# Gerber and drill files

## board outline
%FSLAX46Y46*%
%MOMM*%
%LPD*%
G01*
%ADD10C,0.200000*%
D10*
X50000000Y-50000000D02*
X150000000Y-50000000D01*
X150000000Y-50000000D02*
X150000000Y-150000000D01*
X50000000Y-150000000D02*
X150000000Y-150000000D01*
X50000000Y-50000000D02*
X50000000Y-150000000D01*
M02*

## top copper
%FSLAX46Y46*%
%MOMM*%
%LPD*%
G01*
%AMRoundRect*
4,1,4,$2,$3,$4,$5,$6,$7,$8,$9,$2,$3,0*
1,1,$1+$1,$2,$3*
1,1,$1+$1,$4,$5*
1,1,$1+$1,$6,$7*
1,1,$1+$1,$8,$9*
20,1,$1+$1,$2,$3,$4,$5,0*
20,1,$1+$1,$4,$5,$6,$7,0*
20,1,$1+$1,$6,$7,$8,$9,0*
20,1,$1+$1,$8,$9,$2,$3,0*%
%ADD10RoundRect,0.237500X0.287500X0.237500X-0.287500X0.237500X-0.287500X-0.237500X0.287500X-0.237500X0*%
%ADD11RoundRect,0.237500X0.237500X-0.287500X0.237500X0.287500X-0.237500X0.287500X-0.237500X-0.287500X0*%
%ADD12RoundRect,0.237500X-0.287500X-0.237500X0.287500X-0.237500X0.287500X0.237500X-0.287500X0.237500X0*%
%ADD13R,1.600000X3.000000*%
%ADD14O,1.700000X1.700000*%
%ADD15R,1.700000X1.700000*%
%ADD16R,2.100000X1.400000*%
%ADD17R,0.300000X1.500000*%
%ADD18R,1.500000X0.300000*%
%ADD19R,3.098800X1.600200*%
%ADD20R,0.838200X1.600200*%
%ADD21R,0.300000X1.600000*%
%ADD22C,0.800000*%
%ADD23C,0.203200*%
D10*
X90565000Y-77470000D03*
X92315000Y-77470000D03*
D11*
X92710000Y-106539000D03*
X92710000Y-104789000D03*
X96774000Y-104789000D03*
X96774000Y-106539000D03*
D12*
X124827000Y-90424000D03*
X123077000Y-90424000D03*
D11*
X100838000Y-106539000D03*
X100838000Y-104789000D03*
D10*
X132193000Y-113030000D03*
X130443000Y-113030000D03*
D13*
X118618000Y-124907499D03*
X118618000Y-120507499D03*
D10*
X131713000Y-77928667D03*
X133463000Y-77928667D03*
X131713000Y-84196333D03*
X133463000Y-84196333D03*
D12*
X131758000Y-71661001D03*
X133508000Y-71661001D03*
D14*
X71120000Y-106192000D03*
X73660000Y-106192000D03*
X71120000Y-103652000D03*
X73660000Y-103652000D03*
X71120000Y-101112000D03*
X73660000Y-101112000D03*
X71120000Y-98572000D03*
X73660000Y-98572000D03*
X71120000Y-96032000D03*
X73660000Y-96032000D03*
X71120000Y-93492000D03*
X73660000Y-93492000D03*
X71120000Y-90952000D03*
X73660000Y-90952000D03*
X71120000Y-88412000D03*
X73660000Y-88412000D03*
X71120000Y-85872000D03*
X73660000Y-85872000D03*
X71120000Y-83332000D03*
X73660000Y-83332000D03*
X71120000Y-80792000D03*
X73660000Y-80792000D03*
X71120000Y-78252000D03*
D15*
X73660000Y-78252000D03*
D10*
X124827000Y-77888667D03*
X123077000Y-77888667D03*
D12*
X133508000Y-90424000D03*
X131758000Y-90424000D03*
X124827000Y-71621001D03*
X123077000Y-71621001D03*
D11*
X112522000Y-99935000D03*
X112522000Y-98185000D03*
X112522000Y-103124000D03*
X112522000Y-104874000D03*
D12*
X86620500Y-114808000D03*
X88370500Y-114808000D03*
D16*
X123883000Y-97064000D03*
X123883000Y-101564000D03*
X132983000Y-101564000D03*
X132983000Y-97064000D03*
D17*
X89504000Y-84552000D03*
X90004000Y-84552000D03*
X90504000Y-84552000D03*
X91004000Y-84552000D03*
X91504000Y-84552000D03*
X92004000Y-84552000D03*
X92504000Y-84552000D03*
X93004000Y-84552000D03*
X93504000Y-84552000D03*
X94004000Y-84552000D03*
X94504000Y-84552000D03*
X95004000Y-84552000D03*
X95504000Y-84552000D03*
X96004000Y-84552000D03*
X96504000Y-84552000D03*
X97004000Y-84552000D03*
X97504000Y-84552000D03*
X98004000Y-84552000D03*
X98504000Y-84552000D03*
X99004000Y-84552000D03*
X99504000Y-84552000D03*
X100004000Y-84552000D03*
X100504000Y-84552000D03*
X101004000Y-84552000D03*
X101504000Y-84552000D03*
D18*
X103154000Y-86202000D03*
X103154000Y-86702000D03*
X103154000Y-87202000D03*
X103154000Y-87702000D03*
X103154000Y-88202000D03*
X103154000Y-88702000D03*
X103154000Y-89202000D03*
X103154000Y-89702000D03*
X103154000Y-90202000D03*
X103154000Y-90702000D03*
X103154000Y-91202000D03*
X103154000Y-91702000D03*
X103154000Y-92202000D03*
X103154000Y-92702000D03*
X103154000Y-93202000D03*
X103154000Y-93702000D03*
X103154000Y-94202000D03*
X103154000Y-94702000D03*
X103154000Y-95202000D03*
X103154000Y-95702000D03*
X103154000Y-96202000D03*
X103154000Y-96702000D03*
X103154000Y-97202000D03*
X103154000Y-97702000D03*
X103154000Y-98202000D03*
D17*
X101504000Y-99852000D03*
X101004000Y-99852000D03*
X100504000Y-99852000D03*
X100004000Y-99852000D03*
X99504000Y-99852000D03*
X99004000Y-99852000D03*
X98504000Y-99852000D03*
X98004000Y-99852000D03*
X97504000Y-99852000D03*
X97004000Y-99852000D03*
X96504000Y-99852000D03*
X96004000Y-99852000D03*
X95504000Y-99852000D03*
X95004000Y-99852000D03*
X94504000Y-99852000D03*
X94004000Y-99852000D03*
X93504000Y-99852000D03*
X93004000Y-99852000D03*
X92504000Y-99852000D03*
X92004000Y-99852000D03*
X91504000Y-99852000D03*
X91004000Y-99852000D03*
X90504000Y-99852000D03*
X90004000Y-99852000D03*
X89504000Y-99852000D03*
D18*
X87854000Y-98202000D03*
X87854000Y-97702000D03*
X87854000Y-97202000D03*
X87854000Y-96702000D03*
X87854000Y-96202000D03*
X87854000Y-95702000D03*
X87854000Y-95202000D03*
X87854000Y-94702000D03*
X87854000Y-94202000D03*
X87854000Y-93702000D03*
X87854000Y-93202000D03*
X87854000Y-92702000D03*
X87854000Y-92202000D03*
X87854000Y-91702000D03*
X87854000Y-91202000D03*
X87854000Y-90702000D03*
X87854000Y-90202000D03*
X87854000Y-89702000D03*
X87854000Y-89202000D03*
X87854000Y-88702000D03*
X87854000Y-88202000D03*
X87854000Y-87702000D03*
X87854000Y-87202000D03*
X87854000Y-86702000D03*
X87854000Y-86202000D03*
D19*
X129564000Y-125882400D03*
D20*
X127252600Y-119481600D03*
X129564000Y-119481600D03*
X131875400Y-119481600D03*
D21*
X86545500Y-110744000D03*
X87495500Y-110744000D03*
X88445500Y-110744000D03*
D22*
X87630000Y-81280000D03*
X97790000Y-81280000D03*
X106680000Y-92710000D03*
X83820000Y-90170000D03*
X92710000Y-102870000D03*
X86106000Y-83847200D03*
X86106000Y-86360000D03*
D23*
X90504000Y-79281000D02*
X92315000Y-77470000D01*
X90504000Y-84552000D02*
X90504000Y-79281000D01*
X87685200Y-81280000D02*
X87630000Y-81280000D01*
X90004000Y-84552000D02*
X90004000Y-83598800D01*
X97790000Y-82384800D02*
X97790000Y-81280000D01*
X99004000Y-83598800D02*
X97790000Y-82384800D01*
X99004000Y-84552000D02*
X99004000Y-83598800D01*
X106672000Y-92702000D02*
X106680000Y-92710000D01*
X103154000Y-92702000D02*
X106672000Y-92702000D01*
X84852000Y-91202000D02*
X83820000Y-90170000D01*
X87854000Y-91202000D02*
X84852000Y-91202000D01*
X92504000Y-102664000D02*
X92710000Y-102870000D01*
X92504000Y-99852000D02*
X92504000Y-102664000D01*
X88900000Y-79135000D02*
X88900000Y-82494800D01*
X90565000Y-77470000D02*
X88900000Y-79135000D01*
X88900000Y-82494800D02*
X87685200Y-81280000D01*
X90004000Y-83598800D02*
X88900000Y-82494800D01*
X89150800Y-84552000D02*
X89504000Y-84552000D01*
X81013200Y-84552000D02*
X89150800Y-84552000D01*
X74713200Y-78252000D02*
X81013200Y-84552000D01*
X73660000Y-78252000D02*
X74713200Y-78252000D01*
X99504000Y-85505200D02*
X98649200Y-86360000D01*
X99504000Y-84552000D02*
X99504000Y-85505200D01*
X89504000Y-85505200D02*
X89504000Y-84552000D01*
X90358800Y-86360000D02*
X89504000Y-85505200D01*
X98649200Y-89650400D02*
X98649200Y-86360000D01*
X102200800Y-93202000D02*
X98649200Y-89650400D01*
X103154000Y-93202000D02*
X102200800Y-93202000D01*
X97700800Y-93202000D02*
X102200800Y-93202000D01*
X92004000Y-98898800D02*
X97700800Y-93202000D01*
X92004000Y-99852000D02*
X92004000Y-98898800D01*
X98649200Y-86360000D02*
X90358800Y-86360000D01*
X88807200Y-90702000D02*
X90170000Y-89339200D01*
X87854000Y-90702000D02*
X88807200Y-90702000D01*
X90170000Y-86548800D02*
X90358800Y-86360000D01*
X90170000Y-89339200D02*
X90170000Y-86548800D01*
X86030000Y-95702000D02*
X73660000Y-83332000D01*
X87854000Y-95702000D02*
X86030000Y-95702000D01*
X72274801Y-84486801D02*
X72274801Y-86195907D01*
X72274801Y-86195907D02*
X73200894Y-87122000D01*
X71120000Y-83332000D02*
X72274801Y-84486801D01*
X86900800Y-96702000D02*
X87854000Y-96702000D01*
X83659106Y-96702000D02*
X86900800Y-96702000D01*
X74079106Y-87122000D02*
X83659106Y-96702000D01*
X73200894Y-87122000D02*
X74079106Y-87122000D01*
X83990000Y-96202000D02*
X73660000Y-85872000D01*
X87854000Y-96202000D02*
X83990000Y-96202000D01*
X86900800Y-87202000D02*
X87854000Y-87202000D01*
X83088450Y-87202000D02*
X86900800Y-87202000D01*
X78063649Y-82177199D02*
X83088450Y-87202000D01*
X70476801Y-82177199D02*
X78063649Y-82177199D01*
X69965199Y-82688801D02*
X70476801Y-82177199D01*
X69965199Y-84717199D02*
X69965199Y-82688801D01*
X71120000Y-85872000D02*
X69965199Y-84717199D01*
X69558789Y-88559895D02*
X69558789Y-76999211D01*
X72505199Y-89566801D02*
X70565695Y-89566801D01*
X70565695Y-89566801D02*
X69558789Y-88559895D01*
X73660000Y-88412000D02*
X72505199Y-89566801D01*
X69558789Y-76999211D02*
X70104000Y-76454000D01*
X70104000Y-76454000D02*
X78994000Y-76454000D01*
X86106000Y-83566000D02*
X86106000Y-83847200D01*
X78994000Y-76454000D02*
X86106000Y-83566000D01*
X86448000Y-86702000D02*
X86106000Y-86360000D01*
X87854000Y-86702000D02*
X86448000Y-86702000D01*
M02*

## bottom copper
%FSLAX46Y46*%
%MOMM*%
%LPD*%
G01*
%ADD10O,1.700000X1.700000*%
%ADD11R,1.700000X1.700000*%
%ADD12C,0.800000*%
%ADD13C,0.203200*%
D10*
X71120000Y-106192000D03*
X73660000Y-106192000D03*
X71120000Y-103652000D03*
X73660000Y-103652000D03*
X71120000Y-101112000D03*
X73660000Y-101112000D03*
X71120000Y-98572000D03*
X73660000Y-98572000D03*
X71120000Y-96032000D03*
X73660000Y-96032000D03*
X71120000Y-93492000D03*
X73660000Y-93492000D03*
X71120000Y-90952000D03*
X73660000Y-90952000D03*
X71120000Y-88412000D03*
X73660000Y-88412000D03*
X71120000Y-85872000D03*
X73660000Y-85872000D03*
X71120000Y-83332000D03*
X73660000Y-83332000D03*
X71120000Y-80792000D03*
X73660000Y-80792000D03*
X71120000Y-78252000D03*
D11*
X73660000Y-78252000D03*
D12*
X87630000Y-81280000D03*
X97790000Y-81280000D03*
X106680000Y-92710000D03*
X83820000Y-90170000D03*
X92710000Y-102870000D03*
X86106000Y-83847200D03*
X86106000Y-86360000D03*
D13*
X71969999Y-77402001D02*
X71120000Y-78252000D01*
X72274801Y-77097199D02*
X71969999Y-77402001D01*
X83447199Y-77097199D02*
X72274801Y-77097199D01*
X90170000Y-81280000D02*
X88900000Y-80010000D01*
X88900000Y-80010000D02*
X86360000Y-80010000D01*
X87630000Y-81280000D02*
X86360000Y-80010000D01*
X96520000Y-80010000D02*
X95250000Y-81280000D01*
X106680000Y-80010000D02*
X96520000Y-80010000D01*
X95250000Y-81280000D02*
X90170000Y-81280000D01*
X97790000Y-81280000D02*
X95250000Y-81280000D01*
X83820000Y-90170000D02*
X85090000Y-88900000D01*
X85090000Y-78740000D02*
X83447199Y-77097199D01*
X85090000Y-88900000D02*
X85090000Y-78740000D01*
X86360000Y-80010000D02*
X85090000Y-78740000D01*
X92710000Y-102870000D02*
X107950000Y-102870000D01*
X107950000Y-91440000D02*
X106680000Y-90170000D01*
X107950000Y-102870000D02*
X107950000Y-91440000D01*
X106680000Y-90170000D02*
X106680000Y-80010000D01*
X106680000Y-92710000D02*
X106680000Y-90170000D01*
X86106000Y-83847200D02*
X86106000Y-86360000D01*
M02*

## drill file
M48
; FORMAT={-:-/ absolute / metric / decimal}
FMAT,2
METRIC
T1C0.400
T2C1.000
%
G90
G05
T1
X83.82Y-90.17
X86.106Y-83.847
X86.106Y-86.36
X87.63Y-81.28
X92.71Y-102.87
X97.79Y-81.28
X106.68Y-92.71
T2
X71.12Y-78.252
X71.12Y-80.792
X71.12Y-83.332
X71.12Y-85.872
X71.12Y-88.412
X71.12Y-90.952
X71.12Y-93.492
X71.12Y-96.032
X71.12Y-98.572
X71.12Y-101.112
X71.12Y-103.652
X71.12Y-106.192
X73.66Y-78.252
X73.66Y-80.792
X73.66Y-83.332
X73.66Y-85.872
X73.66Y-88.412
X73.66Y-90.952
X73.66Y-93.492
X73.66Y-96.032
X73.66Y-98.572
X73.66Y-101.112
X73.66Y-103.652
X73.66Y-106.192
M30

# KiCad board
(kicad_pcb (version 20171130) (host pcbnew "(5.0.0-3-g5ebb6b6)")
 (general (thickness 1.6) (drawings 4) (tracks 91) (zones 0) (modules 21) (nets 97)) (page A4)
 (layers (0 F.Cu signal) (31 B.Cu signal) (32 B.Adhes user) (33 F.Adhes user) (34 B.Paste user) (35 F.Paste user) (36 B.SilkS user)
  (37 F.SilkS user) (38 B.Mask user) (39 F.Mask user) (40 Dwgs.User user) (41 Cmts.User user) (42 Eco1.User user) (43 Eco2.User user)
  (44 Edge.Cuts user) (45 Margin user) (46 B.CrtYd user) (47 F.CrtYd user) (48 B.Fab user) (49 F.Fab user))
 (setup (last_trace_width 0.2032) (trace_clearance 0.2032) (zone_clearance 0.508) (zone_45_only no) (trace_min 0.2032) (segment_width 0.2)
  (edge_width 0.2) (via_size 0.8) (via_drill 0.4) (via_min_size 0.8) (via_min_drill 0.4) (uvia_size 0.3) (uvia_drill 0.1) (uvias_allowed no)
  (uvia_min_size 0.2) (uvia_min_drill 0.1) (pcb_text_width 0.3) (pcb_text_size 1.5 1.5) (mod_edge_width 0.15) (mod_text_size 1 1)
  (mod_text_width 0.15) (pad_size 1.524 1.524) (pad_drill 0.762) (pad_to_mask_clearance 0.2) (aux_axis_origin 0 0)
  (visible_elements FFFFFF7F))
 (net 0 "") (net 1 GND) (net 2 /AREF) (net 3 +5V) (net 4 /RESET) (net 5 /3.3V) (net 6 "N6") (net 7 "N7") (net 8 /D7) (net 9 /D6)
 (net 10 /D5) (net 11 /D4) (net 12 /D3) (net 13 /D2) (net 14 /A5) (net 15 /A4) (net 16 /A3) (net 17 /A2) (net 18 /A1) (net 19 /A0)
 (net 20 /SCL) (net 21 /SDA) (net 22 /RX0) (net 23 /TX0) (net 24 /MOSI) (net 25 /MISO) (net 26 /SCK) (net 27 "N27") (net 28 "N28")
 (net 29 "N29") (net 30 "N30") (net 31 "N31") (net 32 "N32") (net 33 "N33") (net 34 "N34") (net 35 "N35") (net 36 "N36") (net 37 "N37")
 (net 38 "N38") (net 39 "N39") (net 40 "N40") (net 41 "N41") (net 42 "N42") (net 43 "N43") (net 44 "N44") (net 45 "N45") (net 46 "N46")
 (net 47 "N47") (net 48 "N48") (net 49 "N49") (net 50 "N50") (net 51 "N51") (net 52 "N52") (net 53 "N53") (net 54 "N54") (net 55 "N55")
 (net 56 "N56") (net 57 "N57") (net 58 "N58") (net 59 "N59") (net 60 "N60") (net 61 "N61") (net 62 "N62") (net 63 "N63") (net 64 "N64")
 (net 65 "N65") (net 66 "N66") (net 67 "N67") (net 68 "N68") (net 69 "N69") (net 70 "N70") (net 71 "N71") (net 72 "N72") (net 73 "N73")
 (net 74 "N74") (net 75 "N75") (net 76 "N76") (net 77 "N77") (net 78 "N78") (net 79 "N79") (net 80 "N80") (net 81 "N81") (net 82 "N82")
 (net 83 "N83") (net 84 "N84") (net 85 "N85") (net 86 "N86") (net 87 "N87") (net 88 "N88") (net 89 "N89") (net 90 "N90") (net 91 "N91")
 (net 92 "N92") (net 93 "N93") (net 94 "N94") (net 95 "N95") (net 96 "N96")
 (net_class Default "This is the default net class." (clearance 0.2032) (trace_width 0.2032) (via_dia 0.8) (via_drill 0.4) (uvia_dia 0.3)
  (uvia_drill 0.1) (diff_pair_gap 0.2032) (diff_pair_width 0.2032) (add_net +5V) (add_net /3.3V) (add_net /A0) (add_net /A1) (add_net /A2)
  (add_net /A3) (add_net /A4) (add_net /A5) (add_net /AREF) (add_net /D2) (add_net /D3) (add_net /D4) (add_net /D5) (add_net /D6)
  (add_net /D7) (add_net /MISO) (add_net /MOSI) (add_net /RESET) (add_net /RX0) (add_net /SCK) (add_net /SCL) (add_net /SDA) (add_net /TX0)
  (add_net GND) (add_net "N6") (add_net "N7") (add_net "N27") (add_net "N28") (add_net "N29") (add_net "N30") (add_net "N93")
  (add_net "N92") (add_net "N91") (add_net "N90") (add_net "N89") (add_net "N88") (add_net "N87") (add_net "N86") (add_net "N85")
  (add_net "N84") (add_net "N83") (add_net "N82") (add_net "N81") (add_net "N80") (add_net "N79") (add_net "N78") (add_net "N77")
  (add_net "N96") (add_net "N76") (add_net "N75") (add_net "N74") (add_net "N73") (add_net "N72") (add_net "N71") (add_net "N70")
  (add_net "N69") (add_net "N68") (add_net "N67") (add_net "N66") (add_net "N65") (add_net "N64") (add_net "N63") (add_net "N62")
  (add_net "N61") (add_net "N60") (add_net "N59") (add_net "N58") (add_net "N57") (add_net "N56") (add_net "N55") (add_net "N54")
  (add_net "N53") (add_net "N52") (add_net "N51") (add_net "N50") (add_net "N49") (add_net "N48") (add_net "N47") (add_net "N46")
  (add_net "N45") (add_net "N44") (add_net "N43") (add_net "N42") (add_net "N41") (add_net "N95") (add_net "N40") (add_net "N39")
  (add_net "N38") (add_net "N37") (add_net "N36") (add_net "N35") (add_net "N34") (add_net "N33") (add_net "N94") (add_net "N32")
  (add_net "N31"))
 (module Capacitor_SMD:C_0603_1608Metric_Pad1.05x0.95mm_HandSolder (layer F.Cu) (at 91.44 77.47 180)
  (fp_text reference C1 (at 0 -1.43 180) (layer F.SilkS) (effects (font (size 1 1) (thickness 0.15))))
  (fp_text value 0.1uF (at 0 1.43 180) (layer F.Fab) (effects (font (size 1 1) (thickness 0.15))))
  (pad 2 smd roundrect (at 0.875 0 180) (size 1.05 0.95) (layers F.Cu F.Paste F.Mask) (roundrect_rratio 0.25) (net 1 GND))
  (pad 1 smd roundrect (at -0.875 0 180) (size 1.05 0.95) (layers F.Cu F.Paste F.Mask) (roundrect_rratio 0.25) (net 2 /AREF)))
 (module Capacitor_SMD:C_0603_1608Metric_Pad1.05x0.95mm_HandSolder (layer F.Cu) (at 92.71 105.664 90)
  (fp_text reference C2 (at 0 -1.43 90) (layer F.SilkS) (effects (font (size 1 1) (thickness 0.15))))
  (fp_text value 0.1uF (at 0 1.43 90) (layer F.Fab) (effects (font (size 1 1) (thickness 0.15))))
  (pad 1 smd roundrect (at -0.875 0 90) (size 1.05 0.95) (layers F.Cu F.Paste F.Mask) (roundrect_rratio 0.25) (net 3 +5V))
  (pad 2 smd roundrect (at 0.875 0 90) (size 1.05 0.95) (layers F.Cu F.Paste F.Mask) (roundrect_rratio 0.25) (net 1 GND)))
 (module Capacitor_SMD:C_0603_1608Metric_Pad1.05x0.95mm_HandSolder (layer F.Cu) (at 96.774 105.664 90)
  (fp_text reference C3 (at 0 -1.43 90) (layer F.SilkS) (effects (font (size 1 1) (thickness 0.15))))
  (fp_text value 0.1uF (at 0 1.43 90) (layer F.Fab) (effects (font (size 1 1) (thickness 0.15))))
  (pad 2 smd roundrect (at 0.875 0 90) (size 1.05 0.95) (layers F.Cu F.Paste F.Mask) (roundrect_rratio 0.25) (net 1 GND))
  (pad 1 smd roundrect (at -0.875 0 90) (size 1.05 0.95) (layers F.Cu F.Paste F.Mask) (roundrect_rratio 0.25) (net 3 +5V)))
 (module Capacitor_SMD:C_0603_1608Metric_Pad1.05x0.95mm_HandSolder (layer F.Cu) (at 123.952 90.424)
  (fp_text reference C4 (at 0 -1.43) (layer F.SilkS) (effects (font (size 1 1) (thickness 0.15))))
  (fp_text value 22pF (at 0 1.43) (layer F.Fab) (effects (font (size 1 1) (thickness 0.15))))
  (pad 2 smd roundrect (at 0.875 0) (size 1.05 0.95) (layers F.Cu F.Paste F.Mask) (roundrect_rratio 0.25) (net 1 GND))
  (pad 1 smd roundrect (at -0.875 0) (size 1.05 0.95) (layers F.Cu F.Paste F.Mask) (roundrect_rratio 0.25) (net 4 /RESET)))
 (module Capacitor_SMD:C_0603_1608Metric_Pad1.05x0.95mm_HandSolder (layer F.Cu) (at 100.838 105.664 90)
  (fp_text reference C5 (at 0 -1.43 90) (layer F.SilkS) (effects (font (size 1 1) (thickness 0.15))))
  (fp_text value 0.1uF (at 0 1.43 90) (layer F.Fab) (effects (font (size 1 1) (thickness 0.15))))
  (pad 1 smd roundrect (at -0.875 0 90) (size 1.05 0.95) (layers F.Cu F.Paste F.Mask) (roundrect_rratio 0.25) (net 3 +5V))
  (pad 2 smd roundrect (at 0.875 0 90) (size 1.05 0.95) (layers F.Cu F.Paste F.Mask) (roundrect_rratio 0.25) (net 1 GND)))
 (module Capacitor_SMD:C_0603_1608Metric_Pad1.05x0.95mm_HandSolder (layer F.Cu) (at 131.318 113.03 180)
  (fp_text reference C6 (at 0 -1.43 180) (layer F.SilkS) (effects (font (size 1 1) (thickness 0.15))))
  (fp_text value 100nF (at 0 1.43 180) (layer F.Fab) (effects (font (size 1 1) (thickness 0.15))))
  (pad 1 smd roundrect (at -0.875 0 180) (size 1.05 0.95) (layers F.Cu F.Paste F.Mask) (roundrect_rratio 0.25) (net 3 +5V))
  (pad 2 smd roundrect (at 0.875 0 180) (size 1.05 0.95) (layers F.Cu F.Paste F.Mask) (roundrect_rratio 0.25) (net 1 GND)))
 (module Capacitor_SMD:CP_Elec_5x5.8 (layer F.Cu) (at 118.618 122.707499 270)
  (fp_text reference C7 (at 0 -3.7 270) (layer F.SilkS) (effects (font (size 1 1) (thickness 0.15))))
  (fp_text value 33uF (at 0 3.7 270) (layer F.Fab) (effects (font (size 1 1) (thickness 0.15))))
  (pad 2 smd rect (at 2.2 0 270) (size 3 1.6) (layers F.Cu F.Paste F.Mask) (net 1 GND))
  (pad 1 smd rect (at -2.2 0 270) (size 3 1.6) (layers F.Cu F.Paste F.Mask) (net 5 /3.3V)))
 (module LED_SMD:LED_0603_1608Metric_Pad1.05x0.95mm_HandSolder (layer F.Cu) (at 132.588 77.928667 180)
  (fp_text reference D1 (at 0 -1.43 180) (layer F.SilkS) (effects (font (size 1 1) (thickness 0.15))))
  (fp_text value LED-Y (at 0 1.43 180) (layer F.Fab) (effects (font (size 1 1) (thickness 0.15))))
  (pad 2 smd roundrect (at 0.875 0 180) (size 1.05 0.95) (layers F.Cu F.Paste F.Mask) (roundrect_rratio 0.25) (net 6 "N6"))
  (pad 1 smd roundrect (at -0.875 0 180) (size 1.05 0.95) (layers F.Cu F.Paste F.Mask) (roundrect_rratio 0.25) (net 1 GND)))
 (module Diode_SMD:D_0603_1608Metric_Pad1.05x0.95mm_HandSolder (layer F.Cu) (at 132.588 84.196333 180)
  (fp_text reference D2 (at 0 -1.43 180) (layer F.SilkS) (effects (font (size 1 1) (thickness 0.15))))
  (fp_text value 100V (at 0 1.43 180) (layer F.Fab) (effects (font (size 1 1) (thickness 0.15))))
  (pad 2 smd roundrect (at 0.875 0 180) (size 1.05 0.95) (layers F.Cu F.Paste F.Mask) (roundrect_rratio 0.25) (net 4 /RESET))
  (pad 1 smd roundrect (at -0.875 0 180) (size 1.05 0.95) (layers F.Cu F.Paste F.Mask) (roundrect_rratio 0.25) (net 3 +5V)))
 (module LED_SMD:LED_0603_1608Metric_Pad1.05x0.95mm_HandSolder (layer F.Cu) (at 132.633 71.661001)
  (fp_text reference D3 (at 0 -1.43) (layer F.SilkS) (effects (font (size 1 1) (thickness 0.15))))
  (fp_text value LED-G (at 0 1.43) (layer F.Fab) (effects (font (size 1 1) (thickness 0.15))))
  (pad 1 smd roundrect (at -0.875 0) (size 1.05 0.95) (layers F.Cu F.Paste F.Mask) (roundrect_rratio 0.25) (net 1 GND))
  (pad 2 smd roundrect (at 0.875 0) (size 1.05 0.95) (layers F.Cu F.Paste F.Mask) (roundrect_rratio 0.25) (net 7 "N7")))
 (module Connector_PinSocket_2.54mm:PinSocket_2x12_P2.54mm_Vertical (layer F.Cu) (at 73.66 78.252)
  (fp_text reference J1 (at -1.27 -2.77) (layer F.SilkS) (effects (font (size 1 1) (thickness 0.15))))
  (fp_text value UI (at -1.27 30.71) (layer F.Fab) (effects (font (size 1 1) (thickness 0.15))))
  (pad 24 thru_hole oval (at -2.54 27.94) (size 1.7 1.7) (drill 1) (layers *.Cu *.Mask) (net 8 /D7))
  (pad 23 thru_hole oval (at 0 27.94) (size 1.7 1.7) (drill 1) (layers *.Cu *.Mask) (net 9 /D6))
  (pad 22 thru_hole oval (at -2.54 25.4) (size 1.7 1.7) (drill 1) (layers *.Cu *.Mask) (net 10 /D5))
  (pad 21 thru_hole oval (at 0 25.4) (size 1.7 1.7) (drill 1) (layers *.Cu *.Mask) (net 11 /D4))
  (pad 20 thru_hole oval (at -2.54 22.86) (size 1.7 1.7) (drill 1) (layers *.Cu *.Mask) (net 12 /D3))
  (pad 19 thru_hole oval (at 0 22.86) (size 1.7 1.7) (drill 1) (layers *.Cu *.Mask) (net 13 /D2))
  (pad 18 thru_hole oval (at -2.54 20.32) (size 1.7 1.7) (drill 1) (layers *.Cu *.Mask) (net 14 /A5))
  (pad 17 thru_hole oval (at 0 20.32) (size 1.7 1.7) (drill 1) (layers *.Cu *.Mask) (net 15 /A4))
  (pad 16 thru_hole oval (at -2.54 17.78) (size 1.7 1.7) (drill 1) (layers *.Cu *.Mask) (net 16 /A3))
  (pad 15 thru_hole oval (at 0 17.78) (size 1.7 1.7) (drill 1) (layers *.Cu *.Mask) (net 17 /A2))
  (pad 14 thru_hole oval (at -2.54 15.24) (size 1.7 1.7) (drill 1) (layers *.Cu *.Mask) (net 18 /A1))
  (pad 13 thru_hole oval (at 0 15.24) (size 1.7 1.7) (drill 1) (layers *.Cu *.Mask) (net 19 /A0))
  (pad 12 thru_hole oval (at -2.54 12.7) (size 1.7 1.7) (drill 1) (layers *.Cu *.Mask) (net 2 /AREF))
  (pad 11 thru_hole oval (at 0 12.7) (size 1.7 1.7) (drill 1) (layers *.Cu *.Mask) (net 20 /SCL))
  (pad 10 thru_hole oval (at -2.54 10.16) (size 1.7 1.7) (drill 1) (layers *.Cu *.Mask) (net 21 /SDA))
  (pad 9 thru_hole oval (at 0 10.16) (size 1.7 1.7) (drill 1) (layers *.Cu *.Mask) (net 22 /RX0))
  (pad 8 thru_hole oval (at -2.54 7.62) (size 1.7 1.7) (drill 1) (layers *.Cu *.Mask) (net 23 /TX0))
  (pad 7 thru_hole oval (at 0 7.62) (size 1.7 1.7) (drill 1) (layers *.Cu *.Mask) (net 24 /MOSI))
  (pad 6 thru_hole oval (at -2.54 5.08) (size 1.7 1.7) (drill 1) (layers *.Cu *.Mask) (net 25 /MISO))
  (pad 5 thru_hole oval (at 0 5.08) (size 1.7 1.7) (drill 1) (layers *.Cu *.Mask) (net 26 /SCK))
  (pad 4 thru_hole oval (at -2.54 2.54) (size 1.7 1.7) (drill 1) (layers *.Cu *.Mask) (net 4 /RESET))
  (pad 3 thru_hole oval (at 0 2.54) (size 1.7 1.7) (drill 1) (layers *.Cu *.Mask) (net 5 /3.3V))
  (pad 2 thru_hole oval (at -2.54 0) (size 1.7 1.7) (drill 1) (layers *.Cu *.Mask) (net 1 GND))
  (pad 1 thru_hole rect (at 0 0) (size 1.7 1.7) (drill 1) (layers *.Cu *.Mask) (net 3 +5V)))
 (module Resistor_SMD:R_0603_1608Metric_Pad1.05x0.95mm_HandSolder (layer F.Cu) (at 123.952 77.888667 180)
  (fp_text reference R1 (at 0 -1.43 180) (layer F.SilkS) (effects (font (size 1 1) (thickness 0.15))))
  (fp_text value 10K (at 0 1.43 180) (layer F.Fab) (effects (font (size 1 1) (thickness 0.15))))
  (pad 1 smd roundrect (at -0.875 0 180) (size 1.05 0.95) (layers F.Cu F.Paste F.Mask) (roundrect_rratio 0.25) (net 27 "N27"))
  (pad 2 smd roundrect (at 0.875 0 180) (size 1.05 0.95) (layers F.Cu F.Paste F.Mask) (roundrect_rratio 0.25) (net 6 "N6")))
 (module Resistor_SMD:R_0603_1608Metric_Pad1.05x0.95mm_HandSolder (layer F.Cu) (at 132.633 90.424)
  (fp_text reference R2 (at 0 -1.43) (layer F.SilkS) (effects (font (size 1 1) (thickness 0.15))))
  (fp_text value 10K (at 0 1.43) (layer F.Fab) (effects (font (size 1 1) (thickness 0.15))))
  (pad 2 smd roundrect (at 0.875 0) (size 1.05 0.95) (layers F.Cu F.Paste F.Mask) (roundrect_rratio 0.25) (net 3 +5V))
  (pad 1 smd roundrect (at -0.875 0) (size 1.05 0.95) (layers F.Cu F.Paste F.Mask) (roundrect_rratio 0.25) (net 4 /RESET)))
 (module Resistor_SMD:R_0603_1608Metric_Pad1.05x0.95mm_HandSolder (layer F.Cu) (at 123.952 71.621001)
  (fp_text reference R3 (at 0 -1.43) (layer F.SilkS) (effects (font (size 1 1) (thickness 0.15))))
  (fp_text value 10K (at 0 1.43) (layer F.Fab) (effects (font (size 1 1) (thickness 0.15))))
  (pad 2 smd roundrect (at 0.875 0) (size 1.05 0.95) (layers F.Cu F.Paste F.Mask) (roundrect_rratio 0.25) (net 7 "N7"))
  (pad 1 smd roundrect (at -0.875 0) (size 1.05 0.95) (layers F.Cu F.Paste F.Mask) (roundrect_rratio 0.25) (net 3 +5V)))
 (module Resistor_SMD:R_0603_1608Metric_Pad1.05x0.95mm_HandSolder (layer F.Cu) (at 112.522 99.06 90)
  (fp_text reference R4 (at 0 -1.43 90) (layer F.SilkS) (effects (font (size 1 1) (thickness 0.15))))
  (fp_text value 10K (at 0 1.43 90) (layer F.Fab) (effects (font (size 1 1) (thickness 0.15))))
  (pad 1 smd roundrect (at -0.875 0 90) (size 1.05 0.95) (layers F.Cu F.Paste F.Mask) (roundrect_rratio 0.25) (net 20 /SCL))
  (pad 2 smd roundrect (at 0.875 0 90) (size 1.05 0.95) (layers F.Cu F.Paste F.Mask) (roundrect_rratio 0.25) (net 3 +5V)))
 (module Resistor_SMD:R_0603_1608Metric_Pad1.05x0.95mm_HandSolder (layer F.Cu) (at 112.522 103.999 90)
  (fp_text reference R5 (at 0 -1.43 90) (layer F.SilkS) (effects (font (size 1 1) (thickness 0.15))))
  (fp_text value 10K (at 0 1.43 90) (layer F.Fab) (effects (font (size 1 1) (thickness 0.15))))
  (pad 2 smd roundrect (at 0.875 0 90) (size 1.05 0.95) (layers F.Cu F.Paste F.Mask) (roundrect_rratio 0.25) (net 3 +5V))
  (pad 1 smd roundrect (at -0.875 0 90) (size 1.05 0.95) (layers F.Cu F.Paste F.Mask) (roundrect_rratio 0.25) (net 21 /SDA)))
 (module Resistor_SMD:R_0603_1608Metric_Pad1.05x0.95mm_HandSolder (layer F.Cu) (at 87.4955 114.808)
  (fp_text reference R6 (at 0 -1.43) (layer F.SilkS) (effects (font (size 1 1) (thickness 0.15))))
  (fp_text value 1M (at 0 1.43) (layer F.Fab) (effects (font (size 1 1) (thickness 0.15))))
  (pad 1 smd roundrect (at -0.875 0) (size 1.05 0.95) (layers F.Cu F.Paste F.Mask) (roundrect_rratio 0.25) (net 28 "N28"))
  (pad 2 smd roundrect (at 0.875 0) (size 1.05 0.95) (layers F.Cu F.Paste F.Mask) (roundrect_rratio 0.25) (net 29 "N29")))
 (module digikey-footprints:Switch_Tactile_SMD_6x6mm (layer F.Cu) (at 128.433 99.314)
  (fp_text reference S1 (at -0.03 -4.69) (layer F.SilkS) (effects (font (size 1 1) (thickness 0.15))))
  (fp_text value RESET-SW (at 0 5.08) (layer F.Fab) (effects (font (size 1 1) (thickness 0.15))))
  (pad 1 smd rect (at -4.55 -2.25 270) (size 1.4 2.1) (layers F.Cu F.Paste F.Mask) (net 1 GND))
  (pad 3 smd rect (at -4.55 2.25 270) (size 1.4 2.1) (layers F.Cu F.Paste F.Mask) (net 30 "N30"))
  (pad 4 smd rect (at 4.55 2.25 270) (size 1.4 2.1) (layers F.Cu F.Paste F.Mask) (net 30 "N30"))
  (pad 2 smd rect (at 4.55 -2.25 270) (size 1.4 2.1) (layers F.Cu F.Paste F.Mask) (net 1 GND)))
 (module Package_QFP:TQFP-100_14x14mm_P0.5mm (layer F.Cu) (at 95.504 92.202)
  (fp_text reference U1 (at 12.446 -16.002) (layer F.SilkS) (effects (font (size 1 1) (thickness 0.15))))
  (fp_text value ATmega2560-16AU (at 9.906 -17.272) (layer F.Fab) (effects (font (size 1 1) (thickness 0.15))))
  (pad 100 smd rect (at -6 -7.65) (size 0.3 1.5) (layers F.Cu F.Paste F.Mask) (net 3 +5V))
  (pad 99 smd rect (at -5.5 -7.65) (size 0.3 1.5) (layers F.Cu F.Paste F.Mask) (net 1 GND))
  (pad 98 smd rect (at -5 -7.65) (size 0.3 1.5) (layers F.Cu F.Paste F.Mask) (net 2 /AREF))
  (pad 97 smd rect (at -4.5 -7.65) (size 0.3 1.5) (layers F.Cu F.Paste F.Mask) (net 19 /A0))
  (pad 96 smd rect (at -4 -7.65) (size 0.3 1.5) (layers F.Cu F.Paste F.Mask) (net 18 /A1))
  (pad 95 smd rect (at -3.5 -7.65) (size 0.3 1.5) (layers F.Cu F.Paste F.Mask) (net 17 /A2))
  (pad 94 smd rect (at -3 -7.65) (size 0.3 1.5) (layers F.Cu F.Paste F.Mask) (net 16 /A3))
  (pad 93 smd rect (at -2.5 -7.65) (size 0.3 1.5) (layers F.Cu F.Paste F.Mask) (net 15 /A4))
  (pad 92 smd rect (at -2 -7.65) (size 0.3 1.5) (layers F.Cu F.Paste F.Mask) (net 14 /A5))
  (pad 91 smd rect (at -1.5 -7.65) (size 0.3 1.5) (layers F.Cu F.Paste F.Mask) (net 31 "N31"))
  (pad 90 smd rect (at -1 -7.65) (size 0.3 1.5) (layers F.Cu F.Paste F.Mask) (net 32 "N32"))
  (pad 89 smd rect (at -0.5 -7.65) (size 0.3 1.5) (layers F.Cu F.Paste F.Mask) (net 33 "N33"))
  (pad 88 smd rect (at 0 -7.65) (size 0.3 1.5) (layers F.Cu F.Paste F.Mask) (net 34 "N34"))
  (pad 87 smd rect (at 0.5 -7.65) (size 0.3 1.5) (layers F.Cu F.Paste F.Mask) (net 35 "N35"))
  (pad 86 smd rect (at 1 -7.65) (size 0.3 1.5) (layers F.Cu F.Paste F.Mask) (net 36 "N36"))
  (pad 85 smd rect (at 1.5 -7.65) (size 0.3 1.5) (layers F.Cu F.Paste F.Mask) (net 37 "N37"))
  (pad 84 smd rect (at 2 -7.65) (size 0.3 1.5) (layers F.Cu F.Paste F.Mask) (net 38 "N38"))
  (pad 83 smd rect (at 2.5 -7.65) (size 0.3 1.5) (layers F.Cu F.Paste F.Mask) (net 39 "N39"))
  (pad 82 smd rect (at 3 -7.65) (size 0.3 1.5) (layers F.Cu F.Paste F.Mask) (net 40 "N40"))
  (pad 81 smd rect (at 3.5 -7.65) (size 0.3 1.5) (layers F.Cu F.Paste F.Mask) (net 1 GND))
  (pad 80 smd rect (at 4 -7.65) (size 0.3 1.5) (layers F.Cu F.Paste F.Mask) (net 3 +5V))
  (pad 79 smd rect (at 4.5 -7.65) (size 0.3 1.5) (layers F.Cu F.Paste F.Mask) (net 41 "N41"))
  (pad 78 smd rect (at 5 -7.65) (size 0.3 1.5) (layers F.Cu F.Paste F.Mask) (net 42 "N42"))
  (pad 77 smd rect (at 5.5 -7.65) (size 0.3 1.5) (layers F.Cu F.Paste F.Mask) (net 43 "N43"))
  (pad 76 smd rect (at 6 -7.65) (size 0.3 1.5) (layers F.Cu F.Paste F.Mask) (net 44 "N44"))
  (pad 75 smd rect (at 7.65 -6) (size 1.5 0.3) (layers F.Cu F.Paste F.Mask) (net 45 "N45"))
  (pad 74 smd rect (at 7.65 -5.5) (size 1.5 0.3) (layers F.Cu F.Paste F.Mask) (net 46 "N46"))
  (pad 73 smd rect (at 7.65 -5) (size 1.5 0.3) (layers F.Cu F.Paste F.Mask) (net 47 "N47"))
  (pad 72 smd rect (at 7.65 -4.5) (size 1.5 0.3) (layers F.Cu F.Paste F.Mask) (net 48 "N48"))
  (pad 71 smd rect (at 7.65 -4) (size 1.5 0.3) (layers F.Cu F.Paste F.Mask) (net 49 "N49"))
  (pad 70 smd rect (at 7.65 -3.5) (size 1.5 0.3) (layers F.Cu F.Paste F.Mask) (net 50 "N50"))
  (pad 69 smd rect (at 7.65 -3) (size 1.5 0.3) (layers F.Cu F.Paste F.Mask) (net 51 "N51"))
  (pad 68 smd rect (at 7.65 -2.5) (size 1.5 0.3) (layers F.Cu F.Paste F.Mask) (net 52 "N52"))
  (pad 67 smd rect (at 7.65 -2) (size 1.5 0.3) (layers F.Cu F.Paste F.Mask) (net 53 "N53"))
  (pad 66 smd rect (at 7.65 -1.5) (size 1.5 0.3) (layers F.Cu F.Paste F.Mask) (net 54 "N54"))
  (pad 65 smd rect (at 7.65 -1) (size 1.5 0.3) (layers F.Cu F.Paste F.Mask) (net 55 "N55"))
  (pad 64 smd rect (at 7.65 -0.5) (size 1.5 0.3) (layers F.Cu F.Paste F.Mask) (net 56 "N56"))
  (pad 63 smd rect (at 7.65 0) (size 1.5 0.3) (layers F.Cu F.Paste F.Mask) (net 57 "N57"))
  (pad 62 smd rect (at 7.65 0.5) (size 1.5 0.3) (layers F.Cu F.Paste F.Mask) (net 1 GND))
  (pad 61 smd rect (at 7.65 1) (size 1.5 0.3) (layers F.Cu F.Paste F.Mask) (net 3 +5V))
  (pad 60 smd rect (at 7.65 1.5) (size 1.5 0.3) (layers F.Cu F.Paste F.Mask) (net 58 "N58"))
  (pad 59 smd rect (at 7.65 2) (size 1.5 0.3) (layers F.Cu F.Paste F.Mask) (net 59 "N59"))
  (pad 58 smd rect (at 7.65 2.5) (size 1.5 0.3) (layers F.Cu F.Paste F.Mask) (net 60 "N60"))
  (pad 57 smd rect (at 7.65 3) (size 1.5 0.3) (layers F.Cu F.Paste F.Mask) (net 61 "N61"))
  (pad 56 smd rect (at 7.65 3.5) (size 1.5 0.3) (layers F.Cu F.Paste F.Mask) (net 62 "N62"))
  (pad 55 smd rect (at 7.65 4) (size 1.5 0.3) (layers F.Cu F.Paste F.Mask) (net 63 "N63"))
  (pad 54 smd rect (at 7.65 4.5) (size 1.5 0.3) (layers F.Cu F.Paste F.Mask) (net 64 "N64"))
  (pad 53 smd rect (at 7.65 5) (size 1.5 0.3) (layers F.Cu F.Paste F.Mask) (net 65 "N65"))
  (pad 52 smd rect (at 7.65 5.5) (size 1.5 0.3) (layers F.Cu F.Paste F.Mask) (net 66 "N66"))
  (pad 51 smd rect (at 7.65 6) (size 1.5 0.3) (layers F.Cu F.Paste F.Mask) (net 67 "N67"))
  (pad 50 smd rect (at 6 7.65) (size 0.3 1.5) (layers F.Cu F.Paste F.Mask) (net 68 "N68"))
  (pad 49 smd rect (at 5.5 7.65) (size 0.3 1.5) (layers F.Cu F.Paste F.Mask) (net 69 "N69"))
  (pad 48 smd rect (at 5 7.65) (size 0.3 1.5) (layers F.Cu F.Paste F.Mask) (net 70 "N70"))
  (pad 47 smd rect (at 4.5 7.65) (size 0.3 1.5) (layers F.Cu F.Paste F.Mask) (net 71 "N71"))
  (pad 46 smd rect (at 4 7.65) (size 0.3 1.5) (layers F.Cu F.Paste F.Mask) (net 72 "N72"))
  (pad 45 smd rect (at 3.5 7.65) (size 0.3 1.5) (layers F.Cu F.Paste F.Mask) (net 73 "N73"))
  (pad 44 smd rect (at 3 7.65) (size 0.3 1.5) (layers F.Cu F.Paste F.Mask) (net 21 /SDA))
  (pad 43 smd rect (at 2.5 7.65) (size 0.3 1.5) (layers F.Cu F.Paste F.Mask) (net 20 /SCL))
  (pad 42 smd rect (at 2 7.65) (size 0.3 1.5) (layers F.Cu F.Paste F.Mask) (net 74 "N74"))
  (pad 41 smd rect (at 1.5 7.65) (size 0.3 1.5) (layers F.Cu F.Paste F.Mask) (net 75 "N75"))
  (pad 40 smd rect (at 1 7.65) (size 0.3 1.5) (layers F.Cu F.Paste F.Mask) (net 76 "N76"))
  (pad 39 smd rect (at 0.5 7.65) (size 0.3 1.5) (layers F.Cu F.Paste F.Mask) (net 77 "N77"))
  (pad 38 smd rect (at 0 7.65) (size 0.3 1.5) (layers F.Cu F.Paste F.Mask) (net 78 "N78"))
  (pad 37 smd rect (at -0.5 7.65) (size 0.3 1.5) (layers F.Cu F.Paste F.Mask) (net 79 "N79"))
  (pad 36 smd rect (at -1 7.65) (size 0.3 1.5) (layers F.Cu F.Paste F.Mask) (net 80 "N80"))
  (pad 35 smd rect (at -1.5 7.65) (size 0.3 1.5) (layers F.Cu F.Paste F.Mask) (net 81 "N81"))
  (pad 34 smd rect (at -2 7.65) (size 0.3 1.5) (layers F.Cu F.Paste F.Mask) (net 29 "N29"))
  (pad 33 smd rect (at -2.5 7.65) (size 0.3 1.5) (layers F.Cu F.Paste F.Mask) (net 28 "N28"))
  (pad 32 smd rect (at -3 7.65) (size 0.3 1.5) (layers F.Cu F.Paste F.Mask) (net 1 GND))
  (pad 31 smd rect (at -3.5 7.65) (size 0.3 1.5) (layers F.Cu F.Paste F.Mask) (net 3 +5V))
  (pad 30 smd rect (at -4 7.65) (size 0.3 1.5) (layers F.Cu F.Paste F.Mask) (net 30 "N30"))
  (pad 29 smd rect (at -4.5 7.65) (size 0.3 1.5) (layers F.Cu F.Paste F.Mask) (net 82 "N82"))
  (pad 28 smd rect (at -5 7.65) (size 0.3 1.5) (layers F.Cu F.Paste F.Mask) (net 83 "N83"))
  (pad 27 smd rect (at -5.5 7.65) (size 0.3 1.5) (layers F.Cu F.Paste F.Mask) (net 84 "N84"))
  (pad 26 smd rect (at -6 7.65) (size 0.3 1.5) (layers F.Cu F.Paste F.Mask) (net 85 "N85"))
  (pad 25 smd rect (at -7.65 6) (size 1.5 0.3) (layers F.Cu F.Paste F.Mask) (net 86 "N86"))
  (pad 24 smd rect (at -7.65 5.5) (size 1.5 0.3) (layers F.Cu F.Paste F.Mask) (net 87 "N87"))
  (pad 23 smd rect (at -7.65 5) (size 1.5 0.3) (layers F.Cu F.Paste F.Mask) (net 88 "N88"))
  (pad 22 smd rect (at -7.65 4.5) (size 1.5 0.3) (layers F.Cu F.Paste F.Mask) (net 25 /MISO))
  (pad 21 smd rect (at -7.65 4) (size 1.5 0.3) (layers F.Cu F.Paste F.Mask) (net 24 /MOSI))
  (pad 20 smd rect (at -7.65 3.5) (size 1.5 0.3) (layers F.Cu F.Paste F.Mask) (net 26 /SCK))
  (pad 19 smd rect (at -7.65 3) (size 1.5 0.3) (layers F.Cu F.Paste F.Mask) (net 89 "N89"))
  (pad 18 smd rect (at -7.65 2.5) (size 1.5 0.3) (layers F.Cu F.Paste F.Mask) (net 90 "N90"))
  (pad 17 smd rect (at -7.65 2) (size 1.5 0.3) (layers F.Cu F.Paste F.Mask) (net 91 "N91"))
  (pad 16 smd rect (at -7.65 1.5) (size 1.5 0.3) (layers F.Cu F.Paste F.Mask) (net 8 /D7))
  (pad 15 smd rect (at -7.65 1) (size 1.5 0.3) (layers F.Cu F.Paste F.Mask) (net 9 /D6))
  (pad 14 smd rect (at -7.65 0.5) (size 1.5 0.3) (layers F.Cu F.Paste F.Mask) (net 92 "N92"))
  (pad 13 smd rect (at -7.65 0) (size 1.5 0.3) (layers F.Cu F.Paste F.Mask) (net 27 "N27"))
  (pad 12 smd rect (at -7.65 -0.5) (size 1.5 0.3) (layers F.Cu F.Paste F.Mask) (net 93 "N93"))
  (pad 11 smd rect (at -7.65 -1) (size 1.5 0.3) (layers F.Cu F.Paste F.Mask) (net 1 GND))
  (pad 10 smd rect (at -7.65 -1.5) (size 1.5 0.3) (layers F.Cu F.Paste F.Mask) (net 3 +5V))
  (pad 9 smd rect (at -7.65 -2) (size 1.5 0.3) (layers F.Cu F.Paste F.Mask) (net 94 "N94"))
  (pad 8 smd rect (at -7.65 -2.5) (size 1.5 0.3) (layers F.Cu F.Paste F.Mask) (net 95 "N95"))
  (pad 7 smd rect (at -7.65 -3) (size 1.5 0.3) (layers F.Cu F.Paste F.Mask) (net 12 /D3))
  (pad 6 smd rect (at -7.65 -3.5) (size 1.5 0.3) (layers F.Cu F.Paste F.Mask) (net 13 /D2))
  (pad 5 smd rect (at -7.65 -4) (size 1.5 0.3) (layers F.Cu F.Paste F.Mask) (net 10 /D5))
  (pad 4 smd rect (at -7.65 -4.5) (size 1.5 0.3) (layers F.Cu F.Paste F.Mask) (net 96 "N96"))
  (pad 3 smd rect (at -7.65 -5) (size 1.5 0.3) (layers F.Cu F.Paste F.Mask) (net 23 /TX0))
  (pad 2 smd rect (at -7.65 -5.5) (size 1.5 0.3) (layers F.Cu F.Paste F.Mask) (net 22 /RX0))
  (pad 1 smd rect (at -7.65 -6) (size 1.5 0.3) (layers F.Cu F.Paste F.Mask) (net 11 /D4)))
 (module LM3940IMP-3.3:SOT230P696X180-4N (layer F.Cu) (at 129.564 122.682 270)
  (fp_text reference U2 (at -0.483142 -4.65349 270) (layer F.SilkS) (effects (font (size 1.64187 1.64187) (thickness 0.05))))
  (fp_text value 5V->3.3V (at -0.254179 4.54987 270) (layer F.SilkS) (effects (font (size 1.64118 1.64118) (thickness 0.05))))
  (pad 4 smd rect (at 3.2004 0 270) (size 1.6002 3.0988) (layers F.Cu F.Paste F.Mask) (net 1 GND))
  (pad 3 smd rect (at -3.2004 2.3114 270) (size 1.6002 0.8382) (layers F.Cu F.Paste F.Mask) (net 5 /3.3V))
  (pad 2 smd rect (at -3.2004 0 270) (size 1.6002 0.8382) (layers F.Cu F.Paste F.Mask) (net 1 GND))
  (pad 1 smd rect (at -3.2004 -2.3114 270) (size 1.6002 0.8382) (layers F.Cu F.Paste F.Mask) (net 3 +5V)))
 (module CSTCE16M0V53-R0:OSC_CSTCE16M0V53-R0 (layer F.Cu) (at 87.4955 110.744 180)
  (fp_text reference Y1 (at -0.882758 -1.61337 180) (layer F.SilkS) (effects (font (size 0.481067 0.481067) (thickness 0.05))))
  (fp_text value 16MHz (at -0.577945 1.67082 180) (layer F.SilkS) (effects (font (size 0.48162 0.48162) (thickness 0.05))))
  (pad 3 smd rect (at 0.95 0 270) (size 1.6 0.3) (layers F.Cu F.Paste F.Mask) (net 28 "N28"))
  (pad 2 smd rect (at 0 0 270) (size 1.6 0.3) (layers F.Cu F.Paste F.Mask) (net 1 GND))
  (pad 1 smd rect (at -0.95 0 270) (size 1.6 0.3) (layers F.Cu F.Paste F.Mask) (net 29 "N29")))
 (gr_line (start 50 50) (end 150 50) (layer Edge.Cuts) (width 0.2))
 (gr_line (start 150 50) (end 150 150) (layer Edge.Cuts) (width 0.2))
 (gr_line (start 50 150) (end 150 150) (layer Edge.Cuts) (width 0.2))
 (gr_line (start 50 50) (end 50 150) (layer Edge.Cuts) (width 0.2))
 (segment (start 90.504 79.281) (end 92.315 77.47) (width 0.2032) (layer F.Cu) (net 2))
 (segment (start 90.504 84.552) (end 90.504 79.281) (width 0.2032) (layer F.Cu) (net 2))
 (segment (start 87.6852 81.28) (end 87.63 81.28) (width 0.2032) (layer F.Cu) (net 1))
 (via (at 87.63 81.28) (size 0.8) (drill 0.4) (layers F.Cu B.Cu) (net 1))
 (segment (start 90.004 84.552) (end 90.004 83.5988) (width 0.2032) (layer F.Cu) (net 1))
 (segment (start 71.969999 77.402001) (end 71.12 78.252) (width 0.2032) (layer B.Cu) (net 1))
 (segment (start 72.274801 77.097199) (end 71.969999 77.402001) (width 0.2032) (layer B.Cu) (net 1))
 (segment (start 83.447199 77.097199) (end 72.274801 77.097199) (width 0.2032) (layer B.Cu) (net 1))
 (via (at 97.79 81.28) (size 0.8) (drill 0.4) (layers F.Cu B.Cu) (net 1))
 (segment (start 97.79 82.3848) (end 97.79 81.28) (width 0.2032) (layer F.Cu) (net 1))
 (segment (start 99.004 83.5988) (end 97.79 82.3848) (width 0.2032) (layer F.Cu) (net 1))
 (segment (start 99.004 84.552) (end 99.004 83.5988) (width 0.2032) (layer F.Cu) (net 1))
 (segment (start 90.17 81.28) (end 88.9 80.01) (width 0.2032) (layer B.Cu) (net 1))
 (segment (start 88.9 80.01) (end 86.36 80.01) (width 0.2032) (layer B.Cu) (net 1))
 (segment (start 87.63 81.28) (end 86.36 80.01) (width 0.2032) (layer B.Cu) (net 1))
 (via (at 106.68 92.71) (size 0.8) (drill 0.4) (layers F.Cu B.Cu) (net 1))
 (segment (start 106.672 92.702) (end 106.68 92.71) (width 0.2032) (layer F.Cu) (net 1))
 (segment (start 103.154 92.702) (end 106.672 92.702) (width 0.2032) (layer F.Cu) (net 1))
 (segment (start 96.52 80.01) (end 95.25 81.28) (width 0.2032) (layer B.Cu) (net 1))
 (segment (start 106.68 80.01) (end 96.52 80.01) (width 0.2032) (layer B.Cu) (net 1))
 (segment (start 95.25 81.28) (end 90.17 81.28) (width 0.2032) (layer B.Cu) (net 1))
 (segment (start 97.79 81.28) (end 95.25 81.28) (width 0.2032) (layer B.Cu) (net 1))
 (via (at 83.82 90.17) (size 0.8) (drill 0.4) (layers F.Cu B.Cu) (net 1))
 (segment (start 84.852 91.202) (end 83.82 90.17) (width 0.2032) (layer F.Cu) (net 1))
 (segment (start 87.854 91.202) (end 84.852 91.202) (width 0.2032) (layer F.Cu) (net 1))
 (segment (start 83.82 90.17) (end 85.09 88.9) (width 0.2032) (layer B.Cu) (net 1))
 (segment (start 85.09 78.74) (end 83.447199 77.097199) (width 0.2032) (layer B.Cu) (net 1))
 (segment (start 85.09 88.9) (end 85.09 78.74) (width 0.2032) (layer B.Cu) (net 1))
 (segment (start 86.36 80.01) (end 85.09 78.74) (width 0.2032) (layer B.Cu) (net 1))
 (via (at 92.71 102.87) (size 0.8) (drill 0.4) (layers F.Cu B.Cu) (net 1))
 (segment (start 92.504 102.664) (end 92.71 102.87) (width 0.2032) (layer F.Cu) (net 1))
 (segment (start 92.504 99.852) (end 92.504 102.664) (width 0.2032) (layer F.Cu) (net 1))
 (segment (start 92.71 102.87) (end 107.95 102.87) (width 0.2032) (layer B.Cu) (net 1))
 (segment (start 107.95 91.44) (end 106.68 90.17) (width 0.2032) (layer B.Cu) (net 1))
 (segment (start 107.95 102.87) (end 107.95 91.44) (width 0.2032) (layer B.Cu) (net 1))
 (segment (start 106.68 90.17) (end 106.68 80.01) (width 0.2032) (layer B.Cu) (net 1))
 (segment (start 106.68 92.71) (end 106.68 90.17) (width 0.2032) (layer B.Cu) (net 1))
 (segment (start 88.9 79.135) (end 88.9 82.4948) (width 0.2032) (layer F.Cu) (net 1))
 (segment (start 90.565 77.47) (end 88.9 79.135) (width 0.2032) (layer F.Cu) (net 1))
 (segment (start 88.9 82.4948) (end 87.6852 81.28) (width 0.2032) (layer F.Cu) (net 1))
 (segment (start 90.004 83.5988) (end 88.9 82.4948) (width 0.2032) (layer F.Cu) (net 1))
 (segment (start 89.1508 84.552) (end 89.504 84.552) (width 0.2032) (layer F.Cu) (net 3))
 (segment (start 81.0132 84.552) (end 89.1508 84.552) (width 0.2032) (layer F.Cu) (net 3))
 (segment (start 74.7132 78.252) (end 81.0132 84.552) (width 0.2032) (layer F.Cu) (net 3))
 (segment (start 73.66 78.252) (end 74.7132 78.252) (width 0.2032) (layer F.Cu) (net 3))
 (segment (start 99.504 85.5052) (end 98.6492 86.36) (width 0.2032) (layer F.Cu) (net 3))
 (segment (start 99.504 84.552) (end 99.504 85.5052) (width 0.2032) (layer F.Cu) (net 3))
 (segment (start 89.504 85.5052) (end 89.504 84.552) (width 0.2032) (layer F.Cu) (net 3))
 (segment (start 90.3588 86.36) (end 89.504 85.5052) (width 0.2032) (layer F.Cu) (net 3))
 (segment (start 98.6492 89.6504) (end 98.6492 86.36) (width 0.2032) (layer F.Cu) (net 3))
 (segment (start 102.2008 93.202) (end 98.6492 89.6504) (width 0.2032) (layer F.Cu) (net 3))
 (segment (start 103.154 93.202) (end 102.2008 93.202) (width 0.2032) (layer F.Cu) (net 3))
 (segment (start 97.7008 93.202) (end 102.2008 93.202) (width 0.2032) (layer F.Cu) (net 3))
 (segment (start 92.004 98.8988) (end 97.7008 93.202) (width 0.2032) (layer F.Cu) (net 3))
 (segment (start 92.004 99.852) (end 92.004 98.8988) (width 0.2032) (layer F.Cu) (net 3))
 (segment (start 98.6492 86.36) (end 90.3588 86.36) (width 0.2032) (layer F.Cu) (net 3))
 (segment (start 88.8072 90.702) (end 90.17 89.3392) (width 0.2032) (layer F.Cu) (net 3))
 (segment (start 87.854 90.702) (end 88.8072 90.702) (width 0.2032) (layer F.Cu) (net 3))
 (segment (start 90.17 86.5488) (end 90.3588 86.36) (width 0.2032) (layer F.Cu) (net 3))
 (segment (start 90.17 89.3392) (end 90.17 86.5488) (width 0.2032) (layer F.Cu) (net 3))
 (segment (start 86.03 95.702) (end 73.66 83.332) (width 0.2032) (layer F.Cu) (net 26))
 (segment (start 87.854 95.702) (end 86.03 95.702) (width 0.2032) (layer F.Cu) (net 26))
 (segment (start 72.274801 84.486801) (end 72.274801 86.195907) (width 0.2032) (layer F.Cu) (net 25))
 (segment (start 72.274801 86.195907) (end 73.200894 87.122) (width 0.2032) (layer F.Cu) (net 25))
 (segment (start 71.12 83.332) (end 72.274801 84.486801) (width 0.2032) (layer F.Cu) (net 25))
 (segment (start 86.9008 96.702) (end 87.854 96.702) (width 0.2032) (layer F.Cu) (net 25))
 (segment (start 83.659106 96.702) (end 86.9008 96.702) (width 0.2032) (layer F.Cu) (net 25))
 (segment (start 74.079106 87.122) (end 83.659106 96.702) (width 0.2032) (layer F.Cu) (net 25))
 (segment (start 73.200894 87.122) (end 74.079106 87.122) (width 0.2032) (layer F.Cu) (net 25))
 (segment (start 83.99 96.202) (end 73.66 85.872) (width 0.2032) (layer F.Cu) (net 24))
 (segment (start 87.854 96.202) (end 83.99 96.202) (width 0.2032) (layer F.Cu) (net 24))
 (segment (start 86.9008 87.202) (end 87.854 87.202) (width 0.2032) (layer F.Cu) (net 23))
 (segment (start 83.08845 87.202) (end 86.9008 87.202) (width 0.2032) (layer F.Cu) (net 23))
 (segment (start 78.063649 82.177199) (end 83.08845 87.202) (width 0.2032) (layer F.Cu) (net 23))
 (segment (start 70.476801 82.177199) (end 78.063649 82.177199) (width 0.2032) (layer F.Cu) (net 23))
 (segment (start 69.965199 82.688801) (end 70.476801 82.177199) (width 0.2032) (layer F.Cu) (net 23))
 (segment (start 69.965199 84.717199) (end 69.965199 82.688801) (width 0.2032) (layer F.Cu) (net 23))
 (segment (start 71.12 85.872) (end 69.965199 84.717199) (width 0.2032) (layer F.Cu) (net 23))
 (segment (start 69.558789 88.559895) (end 69.558789 76.999211) (width 0.2032) (layer F.Cu) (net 22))
 (segment (start 72.505199 89.566801) (end 70.565695 89.566801) (width 0.2032) (layer F.Cu) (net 22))
 (segment (start 70.565695 89.566801) (end 69.558789 88.559895) (width 0.2032) (layer F.Cu) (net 22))
 (segment (start 73.66 88.412) (end 72.505199 89.566801) (width 0.2032) (layer F.Cu) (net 22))
 (segment (start 69.558789 76.999211) (end 70.104 76.454) (width 0.2032) (layer F.Cu) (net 22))
 (segment (start 70.104 76.454) (end 78.994 76.454) (width 0.2032) (layer F.Cu) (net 22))
 (via (at 86.106 83.8472) (size 0.8) (drill 0.4) (layers F.Cu B.Cu) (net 22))
 (segment (start 86.106 83.566) (end 86.106 83.8472) (width 0.2032) (layer F.Cu) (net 22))
 (segment (start 78.994 76.454) (end 86.106 83.566) (width 0.2032) (layer F.Cu) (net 22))
 (segment (start 86.106 83.8472) (end 86.106 86.36) (width 0.2032) (layer B.Cu) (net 22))
 (via (at 86.106 86.36) (size 0.8) (drill 0.4) (layers F.Cu B.Cu) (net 22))
 (segment (start 86.448 86.702) (end 86.106 86.36) (width 0.2032) (layer F.Cu) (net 22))
 (segment (start 87.854 86.702) (end 86.448 86.702) (width 0.2032) (layer F.Cu) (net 22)))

